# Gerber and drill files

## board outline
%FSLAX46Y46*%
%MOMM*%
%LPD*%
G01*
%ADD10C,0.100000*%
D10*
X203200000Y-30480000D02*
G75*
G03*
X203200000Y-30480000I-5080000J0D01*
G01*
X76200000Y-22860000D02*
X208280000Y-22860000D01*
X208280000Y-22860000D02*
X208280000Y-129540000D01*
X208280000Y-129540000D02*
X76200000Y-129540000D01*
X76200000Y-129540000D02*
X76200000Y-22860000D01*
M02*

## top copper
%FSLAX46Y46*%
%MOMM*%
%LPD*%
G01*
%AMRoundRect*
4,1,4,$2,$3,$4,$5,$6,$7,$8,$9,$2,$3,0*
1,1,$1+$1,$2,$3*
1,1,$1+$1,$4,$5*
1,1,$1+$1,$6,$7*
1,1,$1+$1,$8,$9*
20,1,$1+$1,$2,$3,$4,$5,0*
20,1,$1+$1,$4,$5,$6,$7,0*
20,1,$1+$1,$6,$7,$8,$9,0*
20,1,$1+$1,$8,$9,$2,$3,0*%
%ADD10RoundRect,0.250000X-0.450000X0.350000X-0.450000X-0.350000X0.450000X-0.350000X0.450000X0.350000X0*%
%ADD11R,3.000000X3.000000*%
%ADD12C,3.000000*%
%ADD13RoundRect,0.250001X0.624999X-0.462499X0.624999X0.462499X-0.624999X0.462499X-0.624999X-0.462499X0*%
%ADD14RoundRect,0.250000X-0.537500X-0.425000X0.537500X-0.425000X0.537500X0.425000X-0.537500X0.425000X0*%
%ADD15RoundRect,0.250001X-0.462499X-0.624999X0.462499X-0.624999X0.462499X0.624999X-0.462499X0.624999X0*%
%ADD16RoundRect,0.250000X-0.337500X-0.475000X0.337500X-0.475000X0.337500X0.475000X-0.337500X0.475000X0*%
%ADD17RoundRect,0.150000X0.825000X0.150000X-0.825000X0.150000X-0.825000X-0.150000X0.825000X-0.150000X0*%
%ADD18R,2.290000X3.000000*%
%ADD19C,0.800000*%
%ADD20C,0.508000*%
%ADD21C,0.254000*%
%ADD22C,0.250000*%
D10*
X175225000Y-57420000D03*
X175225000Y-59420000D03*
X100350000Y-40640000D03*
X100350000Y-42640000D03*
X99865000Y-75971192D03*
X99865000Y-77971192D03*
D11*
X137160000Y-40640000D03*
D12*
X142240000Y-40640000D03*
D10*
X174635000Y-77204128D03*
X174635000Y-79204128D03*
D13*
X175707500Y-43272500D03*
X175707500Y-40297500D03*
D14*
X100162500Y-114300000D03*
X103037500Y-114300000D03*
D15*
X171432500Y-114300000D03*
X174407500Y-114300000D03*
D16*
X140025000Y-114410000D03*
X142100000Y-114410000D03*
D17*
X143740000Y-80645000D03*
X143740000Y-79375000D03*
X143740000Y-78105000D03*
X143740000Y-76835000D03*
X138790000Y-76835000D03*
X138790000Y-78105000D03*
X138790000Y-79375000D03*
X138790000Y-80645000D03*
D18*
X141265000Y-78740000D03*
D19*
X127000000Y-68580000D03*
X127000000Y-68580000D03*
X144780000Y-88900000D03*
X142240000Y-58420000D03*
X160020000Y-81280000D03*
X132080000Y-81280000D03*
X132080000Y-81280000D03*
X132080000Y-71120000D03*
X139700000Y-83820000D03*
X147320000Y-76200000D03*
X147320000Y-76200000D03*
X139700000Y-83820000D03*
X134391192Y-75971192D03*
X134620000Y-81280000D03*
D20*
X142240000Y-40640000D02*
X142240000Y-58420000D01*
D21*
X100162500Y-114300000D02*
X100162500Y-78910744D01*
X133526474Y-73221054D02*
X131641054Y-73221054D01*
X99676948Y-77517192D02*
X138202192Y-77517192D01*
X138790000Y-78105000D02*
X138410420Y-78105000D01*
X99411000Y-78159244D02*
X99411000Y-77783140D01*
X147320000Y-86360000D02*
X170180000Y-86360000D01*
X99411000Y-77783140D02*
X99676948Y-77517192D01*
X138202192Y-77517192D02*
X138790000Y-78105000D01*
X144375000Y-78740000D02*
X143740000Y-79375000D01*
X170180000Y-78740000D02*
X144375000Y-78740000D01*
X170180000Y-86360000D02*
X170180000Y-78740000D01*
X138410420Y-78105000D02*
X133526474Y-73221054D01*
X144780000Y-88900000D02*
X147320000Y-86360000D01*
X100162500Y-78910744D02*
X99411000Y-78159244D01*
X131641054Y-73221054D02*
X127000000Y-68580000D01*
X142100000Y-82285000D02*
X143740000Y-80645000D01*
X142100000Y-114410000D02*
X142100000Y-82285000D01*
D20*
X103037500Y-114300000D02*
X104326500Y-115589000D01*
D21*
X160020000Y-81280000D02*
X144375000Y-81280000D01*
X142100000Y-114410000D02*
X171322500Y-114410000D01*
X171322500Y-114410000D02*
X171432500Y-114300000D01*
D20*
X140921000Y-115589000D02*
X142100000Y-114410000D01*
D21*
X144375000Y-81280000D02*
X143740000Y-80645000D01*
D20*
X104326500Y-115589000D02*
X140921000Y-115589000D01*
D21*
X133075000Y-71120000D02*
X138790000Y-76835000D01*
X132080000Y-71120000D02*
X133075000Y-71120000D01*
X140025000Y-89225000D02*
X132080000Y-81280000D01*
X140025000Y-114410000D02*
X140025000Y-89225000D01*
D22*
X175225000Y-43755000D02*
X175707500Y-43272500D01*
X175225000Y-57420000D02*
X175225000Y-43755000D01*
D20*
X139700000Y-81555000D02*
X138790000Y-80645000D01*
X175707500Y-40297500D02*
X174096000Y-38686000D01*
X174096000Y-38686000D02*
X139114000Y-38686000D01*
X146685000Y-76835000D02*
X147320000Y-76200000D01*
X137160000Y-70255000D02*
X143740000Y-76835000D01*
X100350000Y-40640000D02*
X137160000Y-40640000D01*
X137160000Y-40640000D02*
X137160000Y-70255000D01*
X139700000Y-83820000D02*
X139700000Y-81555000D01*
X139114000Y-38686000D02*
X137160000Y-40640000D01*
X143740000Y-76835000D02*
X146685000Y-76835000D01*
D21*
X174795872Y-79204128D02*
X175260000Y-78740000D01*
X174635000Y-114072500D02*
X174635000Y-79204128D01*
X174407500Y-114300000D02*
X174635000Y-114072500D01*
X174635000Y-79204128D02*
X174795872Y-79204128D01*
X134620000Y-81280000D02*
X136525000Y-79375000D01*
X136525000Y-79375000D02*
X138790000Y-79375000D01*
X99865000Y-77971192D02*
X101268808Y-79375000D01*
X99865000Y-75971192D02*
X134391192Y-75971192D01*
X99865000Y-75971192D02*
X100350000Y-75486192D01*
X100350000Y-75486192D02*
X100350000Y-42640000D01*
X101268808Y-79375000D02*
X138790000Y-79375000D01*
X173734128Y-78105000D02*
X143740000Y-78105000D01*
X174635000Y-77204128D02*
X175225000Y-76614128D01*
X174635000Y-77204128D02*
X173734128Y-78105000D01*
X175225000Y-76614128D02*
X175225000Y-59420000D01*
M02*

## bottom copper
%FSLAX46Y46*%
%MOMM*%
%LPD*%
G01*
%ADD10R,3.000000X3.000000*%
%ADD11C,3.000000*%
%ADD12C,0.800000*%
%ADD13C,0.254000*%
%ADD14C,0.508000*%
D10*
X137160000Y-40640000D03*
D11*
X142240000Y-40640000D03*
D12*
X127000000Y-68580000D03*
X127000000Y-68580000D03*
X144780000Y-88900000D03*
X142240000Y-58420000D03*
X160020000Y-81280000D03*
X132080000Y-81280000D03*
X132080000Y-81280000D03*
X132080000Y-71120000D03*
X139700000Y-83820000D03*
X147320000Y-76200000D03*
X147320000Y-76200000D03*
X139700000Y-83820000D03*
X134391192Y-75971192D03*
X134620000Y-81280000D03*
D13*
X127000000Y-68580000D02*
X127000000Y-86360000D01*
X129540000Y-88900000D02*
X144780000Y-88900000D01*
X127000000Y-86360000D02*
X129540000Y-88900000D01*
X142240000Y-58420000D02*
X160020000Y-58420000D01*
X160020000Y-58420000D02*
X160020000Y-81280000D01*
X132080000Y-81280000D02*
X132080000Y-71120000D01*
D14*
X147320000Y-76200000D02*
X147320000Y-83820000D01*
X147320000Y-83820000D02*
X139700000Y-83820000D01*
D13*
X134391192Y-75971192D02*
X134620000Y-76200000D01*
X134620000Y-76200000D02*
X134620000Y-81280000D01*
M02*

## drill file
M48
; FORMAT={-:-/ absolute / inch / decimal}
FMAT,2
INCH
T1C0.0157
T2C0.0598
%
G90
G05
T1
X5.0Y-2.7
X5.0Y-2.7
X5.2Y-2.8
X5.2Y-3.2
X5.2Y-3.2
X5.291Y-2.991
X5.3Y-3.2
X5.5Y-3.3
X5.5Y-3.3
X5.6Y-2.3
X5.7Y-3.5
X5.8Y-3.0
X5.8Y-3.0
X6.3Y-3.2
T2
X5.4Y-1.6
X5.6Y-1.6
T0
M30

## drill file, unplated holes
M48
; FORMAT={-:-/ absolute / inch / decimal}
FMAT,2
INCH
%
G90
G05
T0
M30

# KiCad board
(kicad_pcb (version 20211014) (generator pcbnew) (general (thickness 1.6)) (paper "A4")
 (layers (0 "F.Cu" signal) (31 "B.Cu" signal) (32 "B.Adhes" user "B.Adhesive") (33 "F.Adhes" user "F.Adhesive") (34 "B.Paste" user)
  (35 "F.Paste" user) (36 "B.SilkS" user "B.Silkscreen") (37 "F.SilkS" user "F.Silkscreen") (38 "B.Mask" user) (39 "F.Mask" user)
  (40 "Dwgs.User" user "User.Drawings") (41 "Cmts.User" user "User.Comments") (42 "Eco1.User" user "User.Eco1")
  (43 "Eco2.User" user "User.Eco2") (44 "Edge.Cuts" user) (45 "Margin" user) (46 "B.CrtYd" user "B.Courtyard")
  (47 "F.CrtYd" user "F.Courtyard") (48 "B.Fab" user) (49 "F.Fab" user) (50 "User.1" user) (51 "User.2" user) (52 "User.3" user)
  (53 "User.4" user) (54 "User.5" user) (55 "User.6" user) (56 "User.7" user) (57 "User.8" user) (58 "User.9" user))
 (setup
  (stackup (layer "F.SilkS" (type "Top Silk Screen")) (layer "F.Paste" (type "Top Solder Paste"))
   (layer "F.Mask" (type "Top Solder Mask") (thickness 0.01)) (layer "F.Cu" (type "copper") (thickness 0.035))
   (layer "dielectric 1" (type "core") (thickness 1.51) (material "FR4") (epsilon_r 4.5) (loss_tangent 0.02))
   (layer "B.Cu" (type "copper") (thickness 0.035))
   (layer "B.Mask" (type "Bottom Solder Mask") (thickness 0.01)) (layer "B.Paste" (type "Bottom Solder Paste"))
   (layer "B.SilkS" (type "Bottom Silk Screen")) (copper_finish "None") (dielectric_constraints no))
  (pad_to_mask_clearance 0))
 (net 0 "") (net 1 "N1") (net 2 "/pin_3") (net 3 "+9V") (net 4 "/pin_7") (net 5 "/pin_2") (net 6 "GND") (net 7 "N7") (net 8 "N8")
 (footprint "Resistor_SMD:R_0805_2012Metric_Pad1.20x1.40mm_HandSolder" (layer "F.Cu") (at 175.225 58.42 -90)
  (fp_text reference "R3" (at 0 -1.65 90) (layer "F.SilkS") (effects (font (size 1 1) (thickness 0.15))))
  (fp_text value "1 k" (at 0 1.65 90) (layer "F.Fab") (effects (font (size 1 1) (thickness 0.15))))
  (pad "1" smd roundrect (at -1 0 270) (size 1.2 1.4) (layers "F.Cu" "F.Paste" "F.Mask") (roundrect_rratio 0.2083333333) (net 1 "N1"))
  (pad "2" smd roundrect (at 1 0 270) (size 1.2 1.4) (layers "F.Cu" "F.Paste" "F.Mask") (roundrect_rratio 0.2083333333) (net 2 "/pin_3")))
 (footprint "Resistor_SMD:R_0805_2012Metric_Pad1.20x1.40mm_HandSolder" (layer "F.Cu") (at 100.35 41.64 -90)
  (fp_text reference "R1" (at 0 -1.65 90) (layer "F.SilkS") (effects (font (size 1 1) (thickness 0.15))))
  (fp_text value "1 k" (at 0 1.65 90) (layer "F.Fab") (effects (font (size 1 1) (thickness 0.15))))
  (pad "1" smd roundrect (at -1 0 270) (size 1.2 1.4) (layers "F.Cu" "F.Paste" "F.Mask") (roundrect_rratio 0.2083333333) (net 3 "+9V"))
  (pad "2" smd roundrect (at 1 0 270) (size 1.2 1.4) (layers "F.Cu" "F.Paste" "F.Mask") (roundrect_rratio 0.2083333333) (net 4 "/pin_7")))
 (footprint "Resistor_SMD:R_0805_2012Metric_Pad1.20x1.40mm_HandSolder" (layer "F.Cu") (at 99.865 76.971192 -90)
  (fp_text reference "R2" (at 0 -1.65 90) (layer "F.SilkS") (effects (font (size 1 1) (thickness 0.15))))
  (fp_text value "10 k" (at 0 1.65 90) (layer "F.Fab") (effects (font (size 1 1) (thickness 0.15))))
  (pad "1" smd roundrect (at -1 0 270) (size 1.2 1.4) (layers "F.Cu" "F.Paste" "F.Mask") (roundrect_rratio 0.2083333333) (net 4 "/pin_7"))
  (pad "2" smd roundrect (at 1 0 270) (size 1.2 1.4) (layers "F.Cu" "F.Paste" "F.Mask") (roundrect_rratio 0.2083333333) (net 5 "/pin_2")))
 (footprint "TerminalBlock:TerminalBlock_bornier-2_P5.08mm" (layer "F.Cu") (at 137.16 40.64)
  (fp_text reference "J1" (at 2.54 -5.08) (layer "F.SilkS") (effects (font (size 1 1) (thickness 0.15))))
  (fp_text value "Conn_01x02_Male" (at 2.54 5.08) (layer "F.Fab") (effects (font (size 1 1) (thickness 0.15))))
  (pad "1" thru_hole rect (at 0 0) (size 3 3) (drill 1.52) (layers *.Cu *.Mask) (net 3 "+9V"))
  (pad "2" thru_hole circle (at 5.08 0) (size 3 3) (drill 1.52) (layers *.Cu *.Mask) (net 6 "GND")))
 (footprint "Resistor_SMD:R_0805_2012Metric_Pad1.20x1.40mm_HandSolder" (layer "F.Cu") (at 174.635 78.204128 -90)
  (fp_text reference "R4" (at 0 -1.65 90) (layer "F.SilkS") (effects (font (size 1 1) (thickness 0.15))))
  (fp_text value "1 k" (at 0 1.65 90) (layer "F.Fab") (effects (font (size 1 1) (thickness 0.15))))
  (pad "1" smd roundrect (at -1 0 270) (size 1.2 1.4) (layers "F.Cu" "F.Paste" "F.Mask") (roundrect_rratio 0.2083333333) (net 2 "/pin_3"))
  (pad "2" smd roundrect (at 1 0 270) (size 1.2 1.4) (layers "F.Cu" "F.Paste" "F.Mask") (roundrect_rratio 0.2083333333) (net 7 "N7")))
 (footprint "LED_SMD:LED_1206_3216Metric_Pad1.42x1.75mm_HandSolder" (layer "F.Cu") (at 175.7075 41.785 90)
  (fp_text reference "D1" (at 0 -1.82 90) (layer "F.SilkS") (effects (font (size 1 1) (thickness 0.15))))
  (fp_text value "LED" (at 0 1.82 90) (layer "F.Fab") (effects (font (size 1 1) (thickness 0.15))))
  (pad "1" smd roundrect (at -1.4875 0 90) (size 1.425 1.75) (layers "F.Cu" "F.Paste" "F.Mask") (roundrect_rratio 0.1754392982) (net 1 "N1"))
  (pad "2" smd roundrect (at 1.4875 0 90) (size 1.425 1.75) (layers "F.Cu" "F.Paste" "F.Mask") (roundrect_rratio 0.1754392982) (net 3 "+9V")))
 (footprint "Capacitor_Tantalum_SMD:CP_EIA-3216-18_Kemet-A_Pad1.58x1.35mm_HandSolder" (layer "F.Cu") (at 101.6 114.3)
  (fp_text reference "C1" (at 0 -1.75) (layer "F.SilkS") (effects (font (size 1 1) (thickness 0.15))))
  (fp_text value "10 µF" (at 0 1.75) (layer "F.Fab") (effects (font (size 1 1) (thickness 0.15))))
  (pad "1" smd roundrect (at -1.4375 0) (size 1.575 1.35) (layers "F.Cu" "F.Paste" "F.Mask") (roundrect_rratio 0.1851851852)
   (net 5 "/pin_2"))
  (pad "2" smd roundrect (at 1.4375 0) (size 1.575 1.35) (layers "F.Cu" "F.Paste" "F.Mask") (roundrect_rratio 0.1851851852) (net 6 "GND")))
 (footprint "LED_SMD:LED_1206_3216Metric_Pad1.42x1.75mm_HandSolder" (layer "F.Cu") (at 172.92 114.3)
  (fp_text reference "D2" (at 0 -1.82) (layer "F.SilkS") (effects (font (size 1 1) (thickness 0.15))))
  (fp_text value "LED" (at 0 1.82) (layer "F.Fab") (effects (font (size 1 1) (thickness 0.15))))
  (pad "1" smd roundrect (at -1.4875 0) (size 1.425 1.75) (layers "F.Cu" "F.Paste" "F.Mask") (roundrect_rratio 0.1754392982) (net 6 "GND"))
  (pad "2" smd roundrect (at 1.4875 0) (size 1.425 1.75) (layers "F.Cu" "F.Paste" "F.Mask") (roundrect_rratio 0.1754392982) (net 7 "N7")))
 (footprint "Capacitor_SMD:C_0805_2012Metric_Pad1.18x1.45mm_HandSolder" (layer "F.Cu") (at 141.0625 114.41)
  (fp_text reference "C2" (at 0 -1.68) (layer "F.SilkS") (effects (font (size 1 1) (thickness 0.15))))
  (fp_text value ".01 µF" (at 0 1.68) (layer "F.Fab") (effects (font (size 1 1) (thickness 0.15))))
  (pad "1" smd roundrect (at -1.0375 0) (size 1.175 1.45) (layers "F.Cu" "F.Paste" "F.Mask") (roundrect_rratio 0.2127659574) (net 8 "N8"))
  (pad "2" smd roundrect (at 1.0375 0) (size 1.175 1.45) (layers "F.Cu" "F.Paste" "F.Mask") (roundrect_rratio 0.2127659574) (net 6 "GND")))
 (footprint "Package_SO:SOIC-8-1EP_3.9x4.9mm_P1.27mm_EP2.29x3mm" (layer "F.Cu") (at 141.265 78.74 180)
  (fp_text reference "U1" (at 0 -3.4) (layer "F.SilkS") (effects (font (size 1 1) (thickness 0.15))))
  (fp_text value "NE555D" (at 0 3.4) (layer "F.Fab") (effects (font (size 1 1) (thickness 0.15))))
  (pad "" smd roundrect (at -0.57 0.75 180) (size 0.92 1.21) (layers "F.Paste") (roundrect_rratio 0.25))
  (pad "" smd roundrect (at 0.57 -0.75 180) (size 0.92 1.21) (layers "F.Paste") (roundrect_rratio 0.25))
  (pad "" smd roundrect (at 0.57 0.75 180) (size 0.92 1.21) (layers "F.Paste") (roundrect_rratio 0.25))
  (pad "" smd roundrect (at -0.57 -0.75 180) (size 0.92 1.21) (layers "F.Paste") (roundrect_rratio 0.25))
  (pad "1" smd roundrect (at -2.475 -1.905 180) (size 1.95 0.6) (layers "F.Cu" "F.Paste" "F.Mask") (roundrect_rratio 0.25) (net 6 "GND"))
  (pad "2" smd roundrect (at -2.475 -0.635 180) (size 1.95 0.6) (layers "F.Cu" "F.Paste" "F.Mask") (roundrect_rratio 0.25) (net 5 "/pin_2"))
  (pad "3" smd roundrect (at -2.475 0.635 180) (size 1.95 0.6) (layers "F.Cu" "F.Paste" "F.Mask") (roundrect_rratio 0.25) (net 2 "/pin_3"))
  (pad "4" smd roundrect (at -2.475 1.905 180) (size 1.95 0.6) (layers "F.Cu" "F.Paste" "F.Mask") (roundrect_rratio 0.25) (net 3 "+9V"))
  (pad "5" smd roundrect (at 2.475 1.905 180) (size 1.95 0.6) (layers "F.Cu" "F.Paste" "F.Mask") (roundrect_rratio 0.25) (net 8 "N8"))
  (pad "6" smd roundrect (at 2.475 0.635 180) (size 1.95 0.6) (layers "F.Cu" "F.Paste" "F.Mask") (roundrect_rratio 0.25) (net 5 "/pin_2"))
  (pad "7" smd roundrect (at 2.475 -0.635 180) (size 1.95 0.6) (layers "F.Cu" "F.Paste" "F.Mask") (roundrect_rratio 0.25) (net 4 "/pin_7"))
  (pad "8" smd roundrect (at 2.475 -1.905 180) (size 1.95 0.6) (layers "F.Cu" "F.Paste" "F.Mask") (roundrect_rratio 0.25) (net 3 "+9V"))
  (pad "9" smd rect (at 0 0 180) (size 2.29 3) (layers "F.Cu" "F.Mask")))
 (gr_circle (center 198.12 30.48) (end 198.12 35.56) (layer "Edge.Cuts") (width 0.1) (fill none))
 (gr_rect (start 76.2 22.86) (end 208.28 129.54) (layer "Edge.Cuts") (width 0.1) (fill none))
 (segment (start 100.1625 114.3) (end 100.1625 78.910744) (width 0.254) (layer "F.Cu") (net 5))
 (segment (start 133.526474 73.221054) (end 131.641054 73.221054) (width 0.254) (layer "F.Cu") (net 5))
 (segment (start 99.676948 77.517192) (end 138.202192 77.517192) (width 0.254) (layer "F.Cu") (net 5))
 (segment (start 138.79 78.105) (end 138.41042 78.105) (width 0.254) (layer "F.Cu") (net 5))
 (segment (start 99.411 78.159244) (end 99.411 77.78314) (width 0.254) (layer "F.Cu") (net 5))
 (segment (start 147.32 86.36) (end 170.18 86.36) (width 0.254) (layer "F.Cu") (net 5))
 (segment (start 99.411 77.78314) (end 99.676948 77.517192) (width 0.254) (layer "F.Cu") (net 5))
 (segment (start 138.202192 77.517192) (end 138.79 78.105) (width 0.254) (layer "F.Cu") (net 5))
 (segment (start 144.375 78.74) (end 143.74 79.375) (width 0.254) (layer "F.Cu") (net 5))
 (segment (start 170.18 78.74) (end 144.375 78.74) (width 0.254) (layer "F.Cu") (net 5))
 (segment (start 170.18 86.36) (end 170.18 78.74) (width 0.254) (layer "F.Cu") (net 5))
 (segment (start 138.41042 78.105) (end 133.526474 73.221054) (width 0.254) (layer "F.Cu") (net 5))
 (segment (start 144.78 88.9) (end 147.32 86.36) (width 0.254) (layer "F.Cu") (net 5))
 (segment (start 100.1625 78.910744) (end 99.411 78.159244) (width 0.254) (layer "F.Cu") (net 5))
 (segment (start 131.641054 73.221054) (end 127 68.58) (width 0.254) (layer "F.Cu") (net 5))
 (via (at 127 68.58) (size 0.8) (drill 0.4) (layers "F.Cu" "B.Cu") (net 5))
 (via (at 127 68.58) (size 0.8) (drill 0.4) (layers "F.Cu" "B.Cu") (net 5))
 (via (at 144.78 88.9) (size 0.8) (drill 0.4) (layers "F.Cu" "B.Cu") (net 5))
 (segment (start 127 68.58) (end 127 86.36) (width 0.254) (layer "B.Cu") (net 5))
 (segment (start 129.54 88.9) (end 144.78 88.9) (width 0.254) (layer "B.Cu") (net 5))
 (segment (start 127 86.36) (end 129.54 88.9) (width 0.254) (layer "B.Cu") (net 5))
 (segment (start 142.1 82.285) (end 143.74 80.645) (width 0.254) (layer "F.Cu") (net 6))
 (segment (start 142.24 40.64) (end 142.24 58.42) (width 0.508) (layer "F.Cu") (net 6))
 (segment (start 142.1 114.41) (end 142.1 82.285) (width 0.254) (layer "F.Cu") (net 6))
 (segment (start 103.0375 114.3) (end 104.3265 115.589) (width 0.508) (layer "F.Cu") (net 6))
 (segment (start 160.02 81.28) (end 144.375 81.28) (width 0.254) (layer "F.Cu") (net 6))
 (segment (start 142.1 114.41) (end 171.3225 114.41) (width 0.254) (layer "F.Cu") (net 6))
 (segment (start 171.3225 114.41) (end 171.4325 114.3) (width 0.254) (layer "F.Cu") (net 6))
 (segment (start 140.921 115.589) (end 142.1 114.41) (width 0.508) (layer "F.Cu") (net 6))
 (segment (start 144.375 81.28) (end 143.74 80.645) (width 0.254) (layer "F.Cu") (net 6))
 (segment (start 104.3265 115.589) (end 140.921 115.589) (width 0.508) (layer "F.Cu") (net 6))
 (via (at 142.24 58.42) (size 0.8) (drill 0.4) (layers "F.Cu" "B.Cu") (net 6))
 (via (at 160.02 81.28) (size 0.8) (drill 0.4) (layers "F.Cu" "B.Cu") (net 6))
 (segment (start 142.24 58.42) (end 160.02 58.42) (width 0.254) (layer "B.Cu") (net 6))
 (segment (start 160.02 58.42) (end 160.02 81.28) (width 0.254) (layer "B.Cu") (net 6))
 (segment (start 133.075 71.12) (end 138.79 76.835) (width 0.254) (layer "F.Cu") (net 8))
 (segment (start 132.08 71.12) (end 133.075 71.12) (width 0.254) (layer "F.Cu") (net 8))
 (segment (start 140.025 89.225) (end 132.08 81.28) (width 0.254) (layer "F.Cu") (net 8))
 (segment (start 140.025 114.41) (end 140.025 89.225) (width 0.254) (layer "F.Cu") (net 8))
 (via (at 132.08 81.28) (size 0.8) (drill 0.4) (layers "F.Cu" "B.Cu") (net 8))
 (via (at 132.08 81.28) (size 0.8) (drill 0.4) (layers "F.Cu" "B.Cu") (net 8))
 (via (at 132.08 71.12) (size 0.8) (drill 0.4) (layers "F.Cu" "B.Cu") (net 8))
 (segment (start 132.08 81.28) (end 132.08 71.12) (width 0.254) (layer "B.Cu") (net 8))
 (segment (start 175.225 43.755) (end 175.7075 43.2725) (width 0.25) (layer "F.Cu") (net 1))
 (segment (start 175.225 57.42) (end 175.225 43.755) (width 0.25) (layer "F.Cu") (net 1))
 (segment (start 139.7 81.555) (end 138.79 80.645) (width 0.508) (layer "F.Cu") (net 3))
 (segment (start 175.7075 40.2975) (end 174.096 38.686) (width 0.508) (layer "F.Cu") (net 3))
 (segment (start 174.096 38.686) (end 139.114 38.686) (width 0.508) (layer "F.Cu") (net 3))
 (segment (start 146.685 76.835) (end 147.32 76.2) (width 0.508) (layer "F.Cu") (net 3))
 (segment (start 137.16 70.255) (end 143.74 76.835) (width 0.508) (layer "F.Cu") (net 3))
 (segment (start 100.35 40.64) (end 137.16 40.64) (width 0.508) (layer "F.Cu") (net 3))
 (segment (start 137.16 40.64) (end 137.16 70.255) (width 0.508) (layer "F.Cu") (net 3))
 (segment (start 139.7 83.82) (end 139.7 81.555) (width 0.508) (layer "F.Cu") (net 3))
 (segment (start 139.114 38.686) (end 137.16 40.64) (width 0.508) (layer "F.Cu") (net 3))
 (segment (start 143.74 76.835) (end 146.685 76.835) (width 0.508) (layer "F.Cu") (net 3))
 (via (at 139.7 83.82) (size 0.8) (drill 0.4) (layers "F.Cu" "B.Cu") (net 3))
 (via (at 147.32 76.2) (size 0.8) (drill 0.4) (layers "F.Cu" "B.Cu") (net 3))
 (via (at 147.32 76.2) (size 0.8) (drill 0.4) (layers "F.Cu" "B.Cu") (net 3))
 (via (at 139.7 83.82) (size 0.8) (drill 0.4) (layers "F.Cu" "B.Cu") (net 3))
 (segment (start 147.32 76.2) (end 147.32 83.82) (width 0.508) (layer "B.Cu") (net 3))
 (segment (start 147.32 83.82) (end 139.7 83.82) (width 0.508) (layer "B.Cu") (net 3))
 (segment (start 174.795872 79.204128) (end 175.26 78.74) (width 0.254) (layer "F.Cu") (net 7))
 (segment (start 174.635 114.0725) (end 174.635 79.204128) (width 0.254) (layer "F.Cu") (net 7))
 (segment (start 174.4075 114.3) (end 174.635 114.0725) (width 0.254) (layer "F.Cu") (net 7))
 (segment (start 174.635 79.204128) (end 174.795872 79.204128) (width 0.254) (layer "F.Cu") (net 7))
 (segment (start 134.62 81.28) (end 136.525 79.375) (width 0.254) (layer "F.Cu") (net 4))
 (segment (start 136.525 79.375) (end 138.79 79.375) (width 0.254) (layer "F.Cu") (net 4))
 (segment (start 99.865 77.971192) (end 101.268808 79.375) (width 0.254) (layer "F.Cu") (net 4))
 (segment (start 99.865 75.971192) (end 134.391192 75.971192) (width 0.254) (layer "F.Cu") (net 4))
 (segment (start 99.865 75.971192) (end 100.35 75.486192) (width 0.254) (layer "F.Cu") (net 4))
 (segment (start 100.35 75.486192) (end 100.35 42.64) (width 0.254) (layer "F.Cu") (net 4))
 (segment (start 101.268808 79.375) (end 138.79 79.375) (width 0.254) (layer "F.Cu") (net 4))
 (via (at 134.391192 75.971192) (size 0.8) (drill 0.4) (layers "F.Cu" "B.Cu") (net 4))
 (via (at 134.62 81.28) (size 0.8) (drill 0.4) (layers "F.Cu" "B.Cu") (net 4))
 (segment (start 134.391192 75.971192) (end 134.62 76.2) (width 0.254) (layer "B.Cu") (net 4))
 (segment (start 134.62 76.2) (end 134.62 81.28) (width 0.254) (layer "B.Cu") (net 4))
 (segment (start 173.734128 78.105) (end 143.74 78.105) (width 0.254) (layer "F.Cu") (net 2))
 (segment (start 174.635 77.204128) (end 175.225 76.614128) (width 0.254) (layer "F.Cu") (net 2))
 (segment (start 174.635 77.204128) (end 173.734128 78.105) (width 0.254) (layer "F.Cu") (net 2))
 (segment (start 175.225 76.614128) (end 175.225 59.42) (width 0.254) (layer "F.Cu") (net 2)))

